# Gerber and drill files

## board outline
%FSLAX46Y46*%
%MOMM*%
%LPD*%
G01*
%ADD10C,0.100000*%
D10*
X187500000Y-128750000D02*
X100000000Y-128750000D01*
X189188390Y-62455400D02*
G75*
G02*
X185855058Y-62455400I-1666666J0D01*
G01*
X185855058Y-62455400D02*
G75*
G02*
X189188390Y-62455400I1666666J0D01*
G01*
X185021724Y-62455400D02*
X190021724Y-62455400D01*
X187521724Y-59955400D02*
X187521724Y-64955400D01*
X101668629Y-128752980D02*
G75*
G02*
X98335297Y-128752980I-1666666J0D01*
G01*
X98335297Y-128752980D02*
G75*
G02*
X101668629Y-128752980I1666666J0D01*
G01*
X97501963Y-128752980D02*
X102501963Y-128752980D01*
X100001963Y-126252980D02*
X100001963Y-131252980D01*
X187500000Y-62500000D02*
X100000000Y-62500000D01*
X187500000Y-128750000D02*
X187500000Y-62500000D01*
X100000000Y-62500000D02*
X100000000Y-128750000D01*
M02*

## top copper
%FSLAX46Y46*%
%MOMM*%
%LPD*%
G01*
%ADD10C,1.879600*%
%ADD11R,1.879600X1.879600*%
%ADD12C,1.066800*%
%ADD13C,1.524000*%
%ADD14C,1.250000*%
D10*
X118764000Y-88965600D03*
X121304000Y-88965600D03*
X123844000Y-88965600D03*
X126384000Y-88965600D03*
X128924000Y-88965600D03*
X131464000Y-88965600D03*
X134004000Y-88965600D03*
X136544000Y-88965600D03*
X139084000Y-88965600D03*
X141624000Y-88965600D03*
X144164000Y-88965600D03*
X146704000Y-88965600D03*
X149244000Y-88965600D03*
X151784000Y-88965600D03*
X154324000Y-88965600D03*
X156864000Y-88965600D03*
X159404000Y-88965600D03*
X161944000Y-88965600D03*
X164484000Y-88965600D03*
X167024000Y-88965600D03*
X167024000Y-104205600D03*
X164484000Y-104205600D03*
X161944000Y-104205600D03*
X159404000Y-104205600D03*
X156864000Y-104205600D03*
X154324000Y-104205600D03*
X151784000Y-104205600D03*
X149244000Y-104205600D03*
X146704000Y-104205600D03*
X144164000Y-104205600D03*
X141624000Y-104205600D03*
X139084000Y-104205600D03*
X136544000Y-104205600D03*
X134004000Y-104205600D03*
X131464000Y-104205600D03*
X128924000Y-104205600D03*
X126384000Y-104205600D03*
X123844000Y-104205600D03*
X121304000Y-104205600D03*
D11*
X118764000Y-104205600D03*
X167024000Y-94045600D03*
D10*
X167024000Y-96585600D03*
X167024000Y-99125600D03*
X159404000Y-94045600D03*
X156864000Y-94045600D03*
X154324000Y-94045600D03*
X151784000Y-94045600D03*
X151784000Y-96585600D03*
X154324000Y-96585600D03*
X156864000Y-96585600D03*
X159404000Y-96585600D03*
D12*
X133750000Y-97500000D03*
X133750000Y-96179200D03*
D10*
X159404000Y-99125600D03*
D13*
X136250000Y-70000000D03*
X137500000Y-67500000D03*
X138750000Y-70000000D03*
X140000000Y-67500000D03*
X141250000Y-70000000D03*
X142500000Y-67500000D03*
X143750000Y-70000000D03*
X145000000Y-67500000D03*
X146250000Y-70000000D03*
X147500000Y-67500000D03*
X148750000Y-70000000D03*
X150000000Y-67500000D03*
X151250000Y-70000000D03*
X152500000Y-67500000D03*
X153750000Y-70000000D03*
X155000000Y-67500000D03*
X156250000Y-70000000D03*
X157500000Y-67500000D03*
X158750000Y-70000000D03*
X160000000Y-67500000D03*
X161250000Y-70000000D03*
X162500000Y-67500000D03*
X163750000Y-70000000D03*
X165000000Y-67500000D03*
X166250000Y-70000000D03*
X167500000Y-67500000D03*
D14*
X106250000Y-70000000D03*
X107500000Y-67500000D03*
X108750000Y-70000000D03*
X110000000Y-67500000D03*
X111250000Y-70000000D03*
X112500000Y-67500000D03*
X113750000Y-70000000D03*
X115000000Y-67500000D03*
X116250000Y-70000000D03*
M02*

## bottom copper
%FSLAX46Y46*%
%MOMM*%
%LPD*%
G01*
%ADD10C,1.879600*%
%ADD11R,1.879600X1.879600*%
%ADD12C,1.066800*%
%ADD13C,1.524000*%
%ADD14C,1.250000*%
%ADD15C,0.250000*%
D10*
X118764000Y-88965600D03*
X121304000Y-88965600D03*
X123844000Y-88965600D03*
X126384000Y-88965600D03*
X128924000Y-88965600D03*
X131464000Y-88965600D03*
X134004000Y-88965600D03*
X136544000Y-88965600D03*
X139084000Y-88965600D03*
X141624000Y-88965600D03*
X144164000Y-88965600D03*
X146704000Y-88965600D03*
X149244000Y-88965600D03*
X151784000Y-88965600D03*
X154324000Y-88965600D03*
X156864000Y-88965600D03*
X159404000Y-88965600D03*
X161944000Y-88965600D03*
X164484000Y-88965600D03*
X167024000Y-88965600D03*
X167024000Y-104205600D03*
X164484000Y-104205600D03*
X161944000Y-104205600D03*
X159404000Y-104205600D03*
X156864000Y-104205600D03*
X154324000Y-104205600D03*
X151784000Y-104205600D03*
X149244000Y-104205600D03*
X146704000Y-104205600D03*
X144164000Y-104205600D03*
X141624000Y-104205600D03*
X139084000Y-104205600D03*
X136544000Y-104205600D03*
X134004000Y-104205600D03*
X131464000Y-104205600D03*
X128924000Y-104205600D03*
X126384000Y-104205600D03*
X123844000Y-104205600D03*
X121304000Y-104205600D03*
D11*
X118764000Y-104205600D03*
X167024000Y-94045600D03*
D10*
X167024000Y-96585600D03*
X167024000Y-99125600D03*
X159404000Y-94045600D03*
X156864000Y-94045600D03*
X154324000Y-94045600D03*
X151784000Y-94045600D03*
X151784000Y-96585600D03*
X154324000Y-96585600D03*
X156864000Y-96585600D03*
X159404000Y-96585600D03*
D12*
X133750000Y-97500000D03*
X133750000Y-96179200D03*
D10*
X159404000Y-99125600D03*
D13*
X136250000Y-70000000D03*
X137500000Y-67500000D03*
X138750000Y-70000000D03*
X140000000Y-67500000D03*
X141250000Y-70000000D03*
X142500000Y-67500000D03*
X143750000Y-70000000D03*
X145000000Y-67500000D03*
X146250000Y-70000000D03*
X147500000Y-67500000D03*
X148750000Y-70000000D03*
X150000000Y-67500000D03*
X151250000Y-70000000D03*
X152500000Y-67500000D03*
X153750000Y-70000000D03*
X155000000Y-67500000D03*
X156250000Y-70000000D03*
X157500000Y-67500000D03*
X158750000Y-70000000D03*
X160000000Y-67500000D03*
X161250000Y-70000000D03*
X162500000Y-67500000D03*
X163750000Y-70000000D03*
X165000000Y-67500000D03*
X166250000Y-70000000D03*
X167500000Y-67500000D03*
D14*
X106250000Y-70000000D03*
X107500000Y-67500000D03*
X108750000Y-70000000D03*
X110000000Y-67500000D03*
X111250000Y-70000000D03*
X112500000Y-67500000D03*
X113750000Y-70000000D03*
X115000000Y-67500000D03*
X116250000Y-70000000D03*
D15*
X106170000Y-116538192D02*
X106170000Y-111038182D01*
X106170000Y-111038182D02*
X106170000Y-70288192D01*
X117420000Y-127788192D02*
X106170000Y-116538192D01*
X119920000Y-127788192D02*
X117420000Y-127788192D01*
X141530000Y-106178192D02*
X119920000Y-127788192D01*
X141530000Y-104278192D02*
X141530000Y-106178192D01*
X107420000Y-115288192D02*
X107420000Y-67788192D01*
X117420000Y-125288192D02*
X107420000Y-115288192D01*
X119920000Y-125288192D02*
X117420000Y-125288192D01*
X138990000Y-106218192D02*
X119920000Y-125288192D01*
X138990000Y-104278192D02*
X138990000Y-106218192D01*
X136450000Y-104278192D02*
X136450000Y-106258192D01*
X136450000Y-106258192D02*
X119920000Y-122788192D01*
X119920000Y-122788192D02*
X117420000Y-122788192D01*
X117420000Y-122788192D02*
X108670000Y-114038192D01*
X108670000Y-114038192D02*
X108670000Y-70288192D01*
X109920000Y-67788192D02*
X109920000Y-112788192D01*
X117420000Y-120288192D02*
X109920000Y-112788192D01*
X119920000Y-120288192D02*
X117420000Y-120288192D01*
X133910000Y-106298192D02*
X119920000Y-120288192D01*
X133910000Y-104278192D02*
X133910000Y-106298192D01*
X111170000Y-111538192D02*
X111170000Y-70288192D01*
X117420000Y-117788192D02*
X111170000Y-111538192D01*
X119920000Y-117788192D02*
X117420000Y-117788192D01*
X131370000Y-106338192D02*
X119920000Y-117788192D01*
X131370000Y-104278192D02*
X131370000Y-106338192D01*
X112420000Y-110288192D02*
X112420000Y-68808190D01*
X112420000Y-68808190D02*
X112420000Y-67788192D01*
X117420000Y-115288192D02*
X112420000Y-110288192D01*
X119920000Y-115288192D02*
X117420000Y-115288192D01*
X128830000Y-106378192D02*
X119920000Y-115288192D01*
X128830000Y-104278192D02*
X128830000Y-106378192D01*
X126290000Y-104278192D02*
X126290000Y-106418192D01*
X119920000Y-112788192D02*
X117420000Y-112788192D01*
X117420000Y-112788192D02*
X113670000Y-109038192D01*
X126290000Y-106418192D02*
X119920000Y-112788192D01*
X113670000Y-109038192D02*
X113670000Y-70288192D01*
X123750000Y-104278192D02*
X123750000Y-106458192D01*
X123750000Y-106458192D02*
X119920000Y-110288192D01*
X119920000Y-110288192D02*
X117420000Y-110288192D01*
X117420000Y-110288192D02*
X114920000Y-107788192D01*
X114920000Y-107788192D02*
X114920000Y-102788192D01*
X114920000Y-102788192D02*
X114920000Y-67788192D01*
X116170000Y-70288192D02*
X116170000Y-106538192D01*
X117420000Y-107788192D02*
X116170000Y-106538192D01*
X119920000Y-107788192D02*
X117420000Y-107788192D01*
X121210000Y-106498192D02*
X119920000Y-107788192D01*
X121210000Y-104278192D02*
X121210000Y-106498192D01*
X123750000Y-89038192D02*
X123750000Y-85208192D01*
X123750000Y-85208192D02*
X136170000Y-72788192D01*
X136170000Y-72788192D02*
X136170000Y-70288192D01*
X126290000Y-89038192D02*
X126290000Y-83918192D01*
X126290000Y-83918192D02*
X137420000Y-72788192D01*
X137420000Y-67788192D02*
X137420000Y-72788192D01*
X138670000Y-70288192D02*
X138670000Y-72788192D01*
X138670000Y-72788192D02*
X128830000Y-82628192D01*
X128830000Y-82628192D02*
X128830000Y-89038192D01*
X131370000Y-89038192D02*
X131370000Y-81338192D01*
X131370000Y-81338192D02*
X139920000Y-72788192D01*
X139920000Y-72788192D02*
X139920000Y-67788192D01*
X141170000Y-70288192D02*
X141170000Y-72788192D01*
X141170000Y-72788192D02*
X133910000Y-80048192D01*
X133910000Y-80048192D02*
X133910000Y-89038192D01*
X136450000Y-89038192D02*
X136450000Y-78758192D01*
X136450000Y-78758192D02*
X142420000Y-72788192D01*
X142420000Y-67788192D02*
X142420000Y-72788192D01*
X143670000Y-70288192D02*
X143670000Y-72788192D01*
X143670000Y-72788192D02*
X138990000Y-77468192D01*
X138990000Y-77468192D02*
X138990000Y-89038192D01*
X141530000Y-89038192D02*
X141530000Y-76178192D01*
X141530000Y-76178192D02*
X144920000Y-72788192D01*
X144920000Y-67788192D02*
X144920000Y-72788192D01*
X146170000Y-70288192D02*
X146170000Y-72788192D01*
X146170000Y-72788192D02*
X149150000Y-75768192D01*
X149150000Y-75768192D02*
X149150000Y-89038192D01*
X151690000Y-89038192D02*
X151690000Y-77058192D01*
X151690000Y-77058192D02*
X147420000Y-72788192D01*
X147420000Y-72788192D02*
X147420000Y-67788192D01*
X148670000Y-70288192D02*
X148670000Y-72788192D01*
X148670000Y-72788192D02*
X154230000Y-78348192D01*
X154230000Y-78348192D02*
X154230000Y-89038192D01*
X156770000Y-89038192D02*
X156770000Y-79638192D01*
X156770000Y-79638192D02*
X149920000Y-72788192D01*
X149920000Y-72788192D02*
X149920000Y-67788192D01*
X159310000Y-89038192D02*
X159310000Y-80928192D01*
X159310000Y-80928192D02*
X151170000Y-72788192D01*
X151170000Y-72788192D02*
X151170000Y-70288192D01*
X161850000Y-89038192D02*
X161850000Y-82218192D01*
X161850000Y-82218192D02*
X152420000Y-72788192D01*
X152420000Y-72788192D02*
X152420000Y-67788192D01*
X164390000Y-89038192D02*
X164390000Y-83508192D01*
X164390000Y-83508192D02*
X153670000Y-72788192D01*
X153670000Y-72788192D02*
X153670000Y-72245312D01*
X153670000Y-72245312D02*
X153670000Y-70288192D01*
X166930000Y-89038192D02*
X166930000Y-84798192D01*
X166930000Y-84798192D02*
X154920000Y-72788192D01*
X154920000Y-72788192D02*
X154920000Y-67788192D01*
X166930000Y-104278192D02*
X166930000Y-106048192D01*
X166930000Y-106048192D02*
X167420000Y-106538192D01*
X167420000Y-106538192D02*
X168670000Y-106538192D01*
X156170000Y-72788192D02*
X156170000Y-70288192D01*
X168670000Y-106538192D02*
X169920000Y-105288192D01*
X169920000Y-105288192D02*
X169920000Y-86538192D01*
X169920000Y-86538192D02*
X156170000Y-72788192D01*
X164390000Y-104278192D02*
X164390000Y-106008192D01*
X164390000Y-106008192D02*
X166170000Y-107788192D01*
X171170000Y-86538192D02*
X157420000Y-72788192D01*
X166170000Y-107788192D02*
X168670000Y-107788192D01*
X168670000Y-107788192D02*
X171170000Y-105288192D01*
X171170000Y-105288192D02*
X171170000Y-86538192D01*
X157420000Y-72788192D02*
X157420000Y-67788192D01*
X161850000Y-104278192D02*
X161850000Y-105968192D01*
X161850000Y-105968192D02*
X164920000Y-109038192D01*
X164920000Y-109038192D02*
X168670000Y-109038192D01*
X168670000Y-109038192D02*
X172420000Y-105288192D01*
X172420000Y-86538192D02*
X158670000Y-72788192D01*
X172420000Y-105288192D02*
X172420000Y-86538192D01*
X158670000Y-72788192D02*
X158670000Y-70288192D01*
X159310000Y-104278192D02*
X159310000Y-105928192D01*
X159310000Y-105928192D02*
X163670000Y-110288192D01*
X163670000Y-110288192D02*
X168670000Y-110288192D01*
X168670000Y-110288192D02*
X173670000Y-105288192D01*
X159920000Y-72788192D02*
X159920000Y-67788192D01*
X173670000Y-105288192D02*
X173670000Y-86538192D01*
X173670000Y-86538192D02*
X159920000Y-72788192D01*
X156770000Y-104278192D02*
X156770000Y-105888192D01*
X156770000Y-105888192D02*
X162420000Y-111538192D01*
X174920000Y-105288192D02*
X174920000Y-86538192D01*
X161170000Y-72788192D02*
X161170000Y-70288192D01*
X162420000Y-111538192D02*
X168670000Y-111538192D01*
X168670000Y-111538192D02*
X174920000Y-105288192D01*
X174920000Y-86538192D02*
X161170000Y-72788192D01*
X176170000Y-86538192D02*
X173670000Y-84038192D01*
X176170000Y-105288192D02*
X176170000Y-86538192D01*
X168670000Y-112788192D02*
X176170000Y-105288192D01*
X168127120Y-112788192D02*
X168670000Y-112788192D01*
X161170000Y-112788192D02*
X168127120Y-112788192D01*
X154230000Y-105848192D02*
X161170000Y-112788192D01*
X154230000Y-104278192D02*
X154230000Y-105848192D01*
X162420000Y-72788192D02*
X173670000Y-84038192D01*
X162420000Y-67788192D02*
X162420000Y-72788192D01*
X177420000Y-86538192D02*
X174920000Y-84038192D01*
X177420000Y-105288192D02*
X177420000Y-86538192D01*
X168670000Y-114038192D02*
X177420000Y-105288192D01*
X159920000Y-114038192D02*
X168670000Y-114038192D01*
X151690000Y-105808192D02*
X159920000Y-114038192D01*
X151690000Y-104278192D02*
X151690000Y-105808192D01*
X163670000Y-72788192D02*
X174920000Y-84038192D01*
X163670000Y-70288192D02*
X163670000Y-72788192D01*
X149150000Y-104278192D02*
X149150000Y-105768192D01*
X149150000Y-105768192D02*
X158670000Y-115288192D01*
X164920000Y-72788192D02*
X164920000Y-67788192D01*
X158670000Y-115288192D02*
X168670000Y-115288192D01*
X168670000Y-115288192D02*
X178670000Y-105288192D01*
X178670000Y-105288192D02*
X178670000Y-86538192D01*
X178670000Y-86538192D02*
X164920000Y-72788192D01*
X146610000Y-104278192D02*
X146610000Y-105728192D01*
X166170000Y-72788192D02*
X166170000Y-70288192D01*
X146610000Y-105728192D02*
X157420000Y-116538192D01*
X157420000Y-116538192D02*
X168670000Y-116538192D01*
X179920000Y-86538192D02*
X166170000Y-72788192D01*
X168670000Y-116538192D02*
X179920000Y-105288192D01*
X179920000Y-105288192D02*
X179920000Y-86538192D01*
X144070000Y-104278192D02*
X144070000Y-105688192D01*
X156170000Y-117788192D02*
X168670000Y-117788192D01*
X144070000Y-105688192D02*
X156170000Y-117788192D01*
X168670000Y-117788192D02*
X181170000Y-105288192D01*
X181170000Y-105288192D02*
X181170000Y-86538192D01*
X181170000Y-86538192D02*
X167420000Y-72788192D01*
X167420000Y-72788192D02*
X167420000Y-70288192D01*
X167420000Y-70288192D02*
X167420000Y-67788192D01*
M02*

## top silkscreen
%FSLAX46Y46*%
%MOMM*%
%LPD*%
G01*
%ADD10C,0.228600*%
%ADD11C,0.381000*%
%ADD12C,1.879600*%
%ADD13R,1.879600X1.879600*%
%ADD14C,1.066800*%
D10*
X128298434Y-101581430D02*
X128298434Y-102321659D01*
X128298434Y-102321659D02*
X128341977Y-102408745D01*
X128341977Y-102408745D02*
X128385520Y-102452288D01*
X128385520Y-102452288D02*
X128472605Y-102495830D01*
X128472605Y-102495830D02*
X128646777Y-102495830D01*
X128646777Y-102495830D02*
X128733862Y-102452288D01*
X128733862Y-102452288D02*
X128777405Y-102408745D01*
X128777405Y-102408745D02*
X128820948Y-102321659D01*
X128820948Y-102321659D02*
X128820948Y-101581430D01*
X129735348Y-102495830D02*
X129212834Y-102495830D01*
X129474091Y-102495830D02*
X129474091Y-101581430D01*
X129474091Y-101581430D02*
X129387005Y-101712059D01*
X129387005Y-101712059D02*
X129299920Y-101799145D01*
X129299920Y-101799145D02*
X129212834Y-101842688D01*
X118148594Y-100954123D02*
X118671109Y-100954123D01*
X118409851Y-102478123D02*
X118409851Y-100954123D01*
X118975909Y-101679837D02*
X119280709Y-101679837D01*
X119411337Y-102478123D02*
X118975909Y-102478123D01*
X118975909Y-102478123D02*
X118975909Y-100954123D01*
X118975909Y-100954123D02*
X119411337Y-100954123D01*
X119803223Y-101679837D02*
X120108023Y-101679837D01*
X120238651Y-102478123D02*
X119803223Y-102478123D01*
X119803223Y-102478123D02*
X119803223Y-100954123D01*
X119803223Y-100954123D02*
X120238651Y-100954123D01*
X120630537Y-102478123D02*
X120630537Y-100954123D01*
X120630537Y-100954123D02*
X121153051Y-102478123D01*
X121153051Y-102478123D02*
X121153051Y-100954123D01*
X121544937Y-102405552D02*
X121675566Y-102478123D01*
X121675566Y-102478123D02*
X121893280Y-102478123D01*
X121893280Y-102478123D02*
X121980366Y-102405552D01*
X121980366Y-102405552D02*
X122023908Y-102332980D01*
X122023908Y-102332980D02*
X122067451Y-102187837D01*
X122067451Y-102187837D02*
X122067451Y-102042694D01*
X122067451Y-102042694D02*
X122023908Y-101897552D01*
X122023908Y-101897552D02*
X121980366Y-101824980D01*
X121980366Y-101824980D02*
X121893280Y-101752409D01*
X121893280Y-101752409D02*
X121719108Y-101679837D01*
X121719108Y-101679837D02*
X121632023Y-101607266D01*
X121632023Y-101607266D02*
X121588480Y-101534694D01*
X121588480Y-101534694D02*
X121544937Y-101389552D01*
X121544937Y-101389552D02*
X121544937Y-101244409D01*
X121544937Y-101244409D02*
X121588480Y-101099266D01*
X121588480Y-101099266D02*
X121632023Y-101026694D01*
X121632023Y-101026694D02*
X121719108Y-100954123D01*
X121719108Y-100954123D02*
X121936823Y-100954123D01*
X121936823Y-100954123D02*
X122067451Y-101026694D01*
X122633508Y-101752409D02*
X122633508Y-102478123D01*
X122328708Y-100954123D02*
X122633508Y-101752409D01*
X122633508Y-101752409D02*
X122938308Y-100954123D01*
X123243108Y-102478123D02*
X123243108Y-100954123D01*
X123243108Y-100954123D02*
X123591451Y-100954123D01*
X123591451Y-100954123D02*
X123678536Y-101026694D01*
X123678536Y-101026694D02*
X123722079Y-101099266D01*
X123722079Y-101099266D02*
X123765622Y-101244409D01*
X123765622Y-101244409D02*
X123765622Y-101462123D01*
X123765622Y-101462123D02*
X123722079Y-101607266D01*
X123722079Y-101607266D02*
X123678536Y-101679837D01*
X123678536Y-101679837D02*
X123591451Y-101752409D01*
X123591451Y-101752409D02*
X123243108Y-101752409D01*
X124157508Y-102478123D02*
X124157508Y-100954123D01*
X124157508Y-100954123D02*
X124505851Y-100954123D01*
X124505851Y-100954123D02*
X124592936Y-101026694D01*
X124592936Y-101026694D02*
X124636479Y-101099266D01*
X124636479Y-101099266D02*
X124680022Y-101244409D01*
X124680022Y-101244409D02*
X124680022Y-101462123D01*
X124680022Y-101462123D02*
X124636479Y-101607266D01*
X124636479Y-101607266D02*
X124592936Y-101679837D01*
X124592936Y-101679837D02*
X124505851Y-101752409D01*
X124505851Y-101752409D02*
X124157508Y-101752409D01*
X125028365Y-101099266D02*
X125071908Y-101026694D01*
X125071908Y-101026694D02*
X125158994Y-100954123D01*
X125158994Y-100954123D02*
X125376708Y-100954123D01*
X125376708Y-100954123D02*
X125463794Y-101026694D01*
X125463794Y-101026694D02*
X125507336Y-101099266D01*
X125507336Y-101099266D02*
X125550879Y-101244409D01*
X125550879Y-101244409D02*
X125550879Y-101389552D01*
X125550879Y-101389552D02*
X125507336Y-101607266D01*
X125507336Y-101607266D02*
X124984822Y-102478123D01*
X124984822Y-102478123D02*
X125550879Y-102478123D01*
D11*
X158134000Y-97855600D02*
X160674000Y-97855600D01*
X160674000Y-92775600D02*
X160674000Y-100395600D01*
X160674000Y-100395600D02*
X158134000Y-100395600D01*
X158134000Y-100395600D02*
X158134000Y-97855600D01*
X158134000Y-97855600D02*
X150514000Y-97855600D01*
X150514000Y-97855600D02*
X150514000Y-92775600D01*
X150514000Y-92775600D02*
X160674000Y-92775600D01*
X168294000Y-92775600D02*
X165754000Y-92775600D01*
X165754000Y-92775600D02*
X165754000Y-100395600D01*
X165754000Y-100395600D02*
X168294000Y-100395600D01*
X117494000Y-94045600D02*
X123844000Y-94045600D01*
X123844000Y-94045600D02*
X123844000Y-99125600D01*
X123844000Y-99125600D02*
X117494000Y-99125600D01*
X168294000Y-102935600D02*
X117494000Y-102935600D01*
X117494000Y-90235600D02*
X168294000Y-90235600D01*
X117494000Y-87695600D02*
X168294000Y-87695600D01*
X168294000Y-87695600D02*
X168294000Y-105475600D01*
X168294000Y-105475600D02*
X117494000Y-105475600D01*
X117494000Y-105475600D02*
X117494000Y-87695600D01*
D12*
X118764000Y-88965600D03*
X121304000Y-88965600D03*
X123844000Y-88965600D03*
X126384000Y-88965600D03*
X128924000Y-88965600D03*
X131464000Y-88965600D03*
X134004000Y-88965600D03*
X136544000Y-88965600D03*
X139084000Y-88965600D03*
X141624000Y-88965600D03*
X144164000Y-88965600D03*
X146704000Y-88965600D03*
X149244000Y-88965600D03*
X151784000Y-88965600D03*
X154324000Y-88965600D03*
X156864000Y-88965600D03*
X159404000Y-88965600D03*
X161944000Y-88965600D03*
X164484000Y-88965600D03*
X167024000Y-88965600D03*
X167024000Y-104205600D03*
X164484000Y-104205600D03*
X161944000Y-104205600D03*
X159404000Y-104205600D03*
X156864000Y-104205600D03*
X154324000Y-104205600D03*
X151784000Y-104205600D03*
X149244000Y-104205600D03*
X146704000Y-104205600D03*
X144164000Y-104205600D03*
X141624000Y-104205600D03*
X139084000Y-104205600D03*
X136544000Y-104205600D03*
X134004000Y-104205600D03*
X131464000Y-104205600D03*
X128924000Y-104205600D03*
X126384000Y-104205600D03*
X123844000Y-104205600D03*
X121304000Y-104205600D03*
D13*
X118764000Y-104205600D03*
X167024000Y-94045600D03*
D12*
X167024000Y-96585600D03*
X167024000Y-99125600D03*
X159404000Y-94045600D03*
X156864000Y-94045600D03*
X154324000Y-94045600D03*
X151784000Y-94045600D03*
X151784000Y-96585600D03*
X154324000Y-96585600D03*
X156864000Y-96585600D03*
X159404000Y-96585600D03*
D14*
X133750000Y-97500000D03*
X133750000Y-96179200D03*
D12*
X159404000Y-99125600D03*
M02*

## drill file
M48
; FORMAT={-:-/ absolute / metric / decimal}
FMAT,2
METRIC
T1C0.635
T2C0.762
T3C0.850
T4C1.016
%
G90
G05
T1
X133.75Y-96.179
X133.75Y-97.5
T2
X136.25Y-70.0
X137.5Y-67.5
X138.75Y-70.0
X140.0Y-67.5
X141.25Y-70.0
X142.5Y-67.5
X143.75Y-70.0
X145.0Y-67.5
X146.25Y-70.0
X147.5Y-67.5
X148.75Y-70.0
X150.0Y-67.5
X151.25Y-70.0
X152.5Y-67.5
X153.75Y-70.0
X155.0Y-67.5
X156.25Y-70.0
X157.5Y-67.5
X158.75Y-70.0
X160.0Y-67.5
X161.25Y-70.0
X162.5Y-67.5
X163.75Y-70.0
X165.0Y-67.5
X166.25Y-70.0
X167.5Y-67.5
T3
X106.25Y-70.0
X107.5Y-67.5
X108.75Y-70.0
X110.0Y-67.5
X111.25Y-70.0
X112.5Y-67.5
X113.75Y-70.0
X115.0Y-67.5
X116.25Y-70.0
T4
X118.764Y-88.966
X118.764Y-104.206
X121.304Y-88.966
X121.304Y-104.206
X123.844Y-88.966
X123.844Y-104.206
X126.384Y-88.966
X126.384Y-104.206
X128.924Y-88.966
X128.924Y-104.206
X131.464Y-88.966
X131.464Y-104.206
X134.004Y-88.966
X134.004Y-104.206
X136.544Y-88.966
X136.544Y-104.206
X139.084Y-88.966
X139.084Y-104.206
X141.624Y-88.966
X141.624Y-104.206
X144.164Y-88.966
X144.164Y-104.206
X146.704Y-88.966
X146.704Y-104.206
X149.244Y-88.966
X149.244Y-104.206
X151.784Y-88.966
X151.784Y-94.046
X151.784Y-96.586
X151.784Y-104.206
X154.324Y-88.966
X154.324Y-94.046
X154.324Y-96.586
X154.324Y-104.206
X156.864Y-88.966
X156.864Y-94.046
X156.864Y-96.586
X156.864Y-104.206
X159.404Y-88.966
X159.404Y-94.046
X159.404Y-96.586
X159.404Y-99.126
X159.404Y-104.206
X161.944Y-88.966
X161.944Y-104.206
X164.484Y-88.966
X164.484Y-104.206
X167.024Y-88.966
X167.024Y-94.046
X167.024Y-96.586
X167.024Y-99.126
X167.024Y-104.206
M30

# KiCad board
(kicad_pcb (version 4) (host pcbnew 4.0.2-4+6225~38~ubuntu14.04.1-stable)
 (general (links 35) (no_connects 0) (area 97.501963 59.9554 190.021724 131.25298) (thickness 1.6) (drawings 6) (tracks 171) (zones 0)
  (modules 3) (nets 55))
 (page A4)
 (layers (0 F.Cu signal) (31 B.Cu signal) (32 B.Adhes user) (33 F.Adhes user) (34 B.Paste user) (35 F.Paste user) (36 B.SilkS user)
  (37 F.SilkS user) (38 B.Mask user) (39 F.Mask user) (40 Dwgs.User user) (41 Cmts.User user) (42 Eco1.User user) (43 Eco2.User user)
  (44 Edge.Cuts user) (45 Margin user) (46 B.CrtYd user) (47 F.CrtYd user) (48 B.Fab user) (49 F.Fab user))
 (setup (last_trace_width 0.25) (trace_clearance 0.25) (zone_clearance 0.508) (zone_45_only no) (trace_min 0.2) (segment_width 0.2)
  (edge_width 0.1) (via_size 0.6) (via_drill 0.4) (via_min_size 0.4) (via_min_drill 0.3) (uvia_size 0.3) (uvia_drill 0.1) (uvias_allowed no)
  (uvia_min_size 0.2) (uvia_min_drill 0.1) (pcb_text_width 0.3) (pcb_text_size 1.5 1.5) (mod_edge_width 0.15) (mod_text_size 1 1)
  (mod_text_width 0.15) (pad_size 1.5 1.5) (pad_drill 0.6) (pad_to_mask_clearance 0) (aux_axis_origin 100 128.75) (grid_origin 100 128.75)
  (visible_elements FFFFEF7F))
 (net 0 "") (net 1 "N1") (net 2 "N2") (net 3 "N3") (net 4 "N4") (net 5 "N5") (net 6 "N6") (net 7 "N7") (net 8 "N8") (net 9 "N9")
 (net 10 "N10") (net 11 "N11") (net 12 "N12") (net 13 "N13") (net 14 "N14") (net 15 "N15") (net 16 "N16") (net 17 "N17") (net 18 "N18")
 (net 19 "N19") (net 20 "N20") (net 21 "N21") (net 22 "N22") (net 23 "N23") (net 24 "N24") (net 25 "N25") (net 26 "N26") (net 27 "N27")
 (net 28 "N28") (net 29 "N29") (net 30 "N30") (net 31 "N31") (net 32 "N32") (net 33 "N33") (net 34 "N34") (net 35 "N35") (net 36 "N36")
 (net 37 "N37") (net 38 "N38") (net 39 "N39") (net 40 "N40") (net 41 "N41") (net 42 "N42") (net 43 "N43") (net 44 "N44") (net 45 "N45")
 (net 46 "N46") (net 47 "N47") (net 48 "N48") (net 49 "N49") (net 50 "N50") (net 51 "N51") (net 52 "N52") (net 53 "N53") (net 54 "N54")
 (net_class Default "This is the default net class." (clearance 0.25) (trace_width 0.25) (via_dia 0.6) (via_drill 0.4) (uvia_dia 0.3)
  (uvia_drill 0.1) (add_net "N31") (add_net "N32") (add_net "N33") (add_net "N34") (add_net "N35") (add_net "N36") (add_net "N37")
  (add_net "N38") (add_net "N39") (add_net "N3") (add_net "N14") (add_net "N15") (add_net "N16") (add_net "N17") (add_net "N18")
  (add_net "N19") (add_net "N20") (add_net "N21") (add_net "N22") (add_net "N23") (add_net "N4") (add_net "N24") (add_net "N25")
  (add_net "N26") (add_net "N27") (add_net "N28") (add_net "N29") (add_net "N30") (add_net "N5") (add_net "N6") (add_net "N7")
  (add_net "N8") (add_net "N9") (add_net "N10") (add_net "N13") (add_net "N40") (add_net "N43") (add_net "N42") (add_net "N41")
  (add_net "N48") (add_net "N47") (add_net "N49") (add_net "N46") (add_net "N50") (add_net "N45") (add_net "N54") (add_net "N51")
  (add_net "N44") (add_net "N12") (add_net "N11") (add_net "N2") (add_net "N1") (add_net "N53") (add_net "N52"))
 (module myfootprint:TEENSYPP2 (layer F.Cu) (at 142.894 96.5856)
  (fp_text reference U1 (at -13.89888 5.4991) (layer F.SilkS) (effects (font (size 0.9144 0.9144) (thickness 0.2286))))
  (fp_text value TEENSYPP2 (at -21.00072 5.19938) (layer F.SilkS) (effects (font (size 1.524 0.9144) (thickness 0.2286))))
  (fp_line (start 15.24 1.27) (end 17.78 1.27) (layer F.SilkS) (width 0.381))
  (fp_line (start 17.78 -3.81) (end 17.78 3.81) (layer F.SilkS) (width 0.381))
  (fp_line (start 17.78 3.81) (end 15.24 3.81) (layer F.SilkS) (width 0.381))
  (fp_line (start 15.24 3.81) (end 15.24 1.27) (layer F.SilkS) (width 0.381))
  (fp_line (start 15.24 1.27) (end 7.62 1.27) (layer F.SilkS) (width 0.381))
  (fp_line (start 7.62 1.27) (end 7.62 -3.81) (layer F.SilkS) (width 0.381))
  (fp_line (start 7.62 -3.81) (end 17.78 -3.81) (layer F.SilkS) (width 0.381))
  (fp_line (start 25.4 -3.81) (end 22.86 -3.81) (layer F.SilkS) (width 0.381))
  (fp_line (start 22.86 -3.81) (end 22.86 3.81) (layer F.SilkS) (width 0.381))
  (fp_line (start 22.86 3.81) (end 25.4 3.81) (layer F.SilkS) (width 0.381))
  (fp_line (start -25.4 -2.54) (end -19.05 -2.54) (layer F.SilkS) (width 0.381))
  (fp_line (start -19.05 -2.54) (end -19.05 2.54) (layer F.SilkS) (width 0.381))
  (fp_line (start -19.05 2.54) (end -25.4 2.54) (layer F.SilkS) (width 0.381))
  (fp_line (start 25.4 6.35) (end -25.4 6.35) (layer F.SilkS) (width 0.381))
  (fp_line (start -25.4 -6.35) (end 25.4 -6.35) (layer F.SilkS) (width 0.381))
  (fp_line (start -25.4 -8.89) (end 25.4 -8.89) (layer F.SilkS) (width 0.381))
  (fp_line (start 25.4 -8.89) (end 25.4 8.89) (layer F.SilkS) (width 0.381))
  (fp_line (start 25.4 8.89) (end -25.4 8.89) (layer F.SilkS) (width 0.381))
  (fp_line (start -25.4 8.89) (end -25.4 -8.89) (layer F.SilkS) (width 0.381))
  (pad 52 thru_hole circle (at -24.13 -7.62) (size 1.8796 1.8796) (drill 1.016) (layers *.Cu *.Mask F.SilkS) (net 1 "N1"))
  (pad 51 thru_hole circle (at -21.59 -7.62) (size 1.8796 1.8796) (drill 1.016) (layers *.Cu *.Mask F.SilkS) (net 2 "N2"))
  (pad 50 thru_hole circle (at -19.05 -7.62) (size 1.8796 1.8796) (drill 1.016) (layers *.Cu *.Mask F.SilkS) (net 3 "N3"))
  (pad 49 thru_hole circle (at -16.51 -7.62) (size 1.8796 1.8796) (drill 1.016) (layers *.Cu *.Mask F.SilkS) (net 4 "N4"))
  (pad 48 thru_hole circle (at -13.97 -7.62) (size 1.8796 1.8796) (drill 1.016) (layers *.Cu *.Mask F.SilkS) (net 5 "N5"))
  (pad 47 thru_hole circle (at -11.43 -7.62) (size 1.8796 1.8796) (drill 1.016) (layers *.Cu *.Mask F.SilkS) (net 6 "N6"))
  (pad 46 thru_hole circle (at -8.89 -7.62) (size 1.8796 1.8796) (drill 1.016) (layers *.Cu *.Mask F.SilkS) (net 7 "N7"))
  (pad 45 thru_hole circle (at -6.35 -7.62) (size 1.8796 1.8796) (drill 1.016) (layers *.Cu *.Mask F.SilkS) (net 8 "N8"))
  (pad 44 thru_hole circle (at -3.81 -7.62) (size 1.8796 1.8796) (drill 1.016) (layers *.Cu *.Mask F.SilkS) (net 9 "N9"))
  (pad 43 thru_hole circle (at -1.27 -7.62) (size 1.8796 1.8796) (drill 1.016) (layers *.Cu *.Mask F.SilkS) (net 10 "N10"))
  (pad 42 thru_hole circle (at 1.27 -7.62) (size 1.8796 1.8796) (drill 1.016) (layers *.Cu *.Mask F.SilkS) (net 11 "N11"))
  (pad 41 thru_hole circle (at 3.81 -7.62) (size 1.8796 1.8796) (drill 1.016) (layers *.Cu *.Mask F.SilkS) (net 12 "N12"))
  (pad 40 thru_hole circle (at 6.35 -7.62) (size 1.8796 1.8796) (drill 1.016) (layers *.Cu *.Mask F.SilkS) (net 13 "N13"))
  (pad 39 thru_hole circle (at 8.89 -7.62) (size 1.8796 1.8796) (drill 1.016) (layers *.Cu *.Mask F.SilkS) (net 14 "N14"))
  (pad 38 thru_hole circle (at 11.43 -7.62) (size 1.8796 1.8796) (drill 1.016) (layers *.Cu *.Mask F.SilkS) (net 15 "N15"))
  (pad 37 thru_hole circle (at 13.97 -7.62) (size 1.8796 1.8796) (drill 1.016) (layers *.Cu *.Mask F.SilkS) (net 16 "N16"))
  (pad 36 thru_hole circle (at 16.51 -7.62) (size 1.8796 1.8796) (drill 1.016) (layers *.Cu *.Mask F.SilkS) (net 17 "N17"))
  (pad 35 thru_hole circle (at 19.05 -7.62) (size 1.8796 1.8796) (drill 1.016) (layers *.Cu *.Mask F.SilkS) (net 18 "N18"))
  (pad 34 thru_hole circle (at 21.59 -7.62) (size 1.8796 1.8796) (drill 1.016) (layers *.Cu *.Mask F.SilkS) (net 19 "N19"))
  (pad 33 thru_hole circle (at 24.13 -7.62) (size 1.8796 1.8796) (drill 1.016) (layers *.Cu *.Mask F.SilkS) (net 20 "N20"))
  (pad 20 thru_hole circle (at 24.13 7.62) (size 1.8796 1.8796) (drill 1.016) (layers *.Cu *.Mask F.SilkS) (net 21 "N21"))
  (pad 19 thru_hole circle (at 21.59 7.62) (size 1.8796 1.8796) (drill 1.016) (layers *.Cu *.Mask F.SilkS) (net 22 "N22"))
  (pad 18 thru_hole circle (at 19.05 7.62) (size 1.8796 1.8796) (drill 1.016) (layers *.Cu *.Mask F.SilkS) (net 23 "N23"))
  (pad 17 thru_hole circle (at 16.51 7.62) (size 1.8796 1.8796) (drill 1.016) (layers *.Cu *.Mask F.SilkS) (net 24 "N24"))
  (pad 16 thru_hole circle (at 13.97 7.62) (size 1.8796 1.8796) (drill 1.016) (layers *.Cu *.Mask F.SilkS) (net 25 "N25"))
  (pad 15 thru_hole circle (at 11.43 7.62) (size 1.8796 1.8796) (drill 1.016) (layers *.Cu *.Mask F.SilkS) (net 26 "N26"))
  (pad 14 thru_hole circle (at 8.89 7.62) (size 1.8796 1.8796) (drill 1.016) (layers *.Cu *.Mask F.SilkS) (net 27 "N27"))
  (pad 13 thru_hole circle (at 6.35 7.62) (size 1.8796 1.8796) (drill 1.016) (layers *.Cu *.Mask F.SilkS) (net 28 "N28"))
  (pad 12 thru_hole circle (at 3.81 7.62) (size 1.8796 1.8796) (drill 1.016) (layers *.Cu *.Mask F.SilkS) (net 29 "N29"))
  (pad 11 thru_hole circle (at 1.27 7.62) (size 1.8796 1.8796) (drill 1.016) (layers *.Cu *.Mask F.SilkS) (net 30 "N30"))
  (pad 10 thru_hole circle (at -1.27 7.62) (size 1.8796 1.8796) (drill 1.016) (layers *.Cu *.Mask F.SilkS) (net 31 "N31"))
  (pad 9 thru_hole circle (at -3.81 7.62) (size 1.8796 1.8796) (drill 1.016) (layers *.Cu *.Mask F.SilkS) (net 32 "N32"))
  (pad 8 thru_hole circle (at -6.35 7.62) (size 1.8796 1.8796) (drill 1.016) (layers *.Cu *.Mask F.SilkS) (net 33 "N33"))
  (pad 7 thru_hole circle (at -8.89 7.62) (size 1.8796 1.8796) (drill 1.016) (layers *.Cu *.Mask F.SilkS) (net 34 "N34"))
  (pad 6 thru_hole circle (at -11.43 7.62) (size 1.8796 1.8796) (drill 1.016) (layers *.Cu *.Mask F.SilkS) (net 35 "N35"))
  (pad 5 thru_hole circle (at -13.97 7.62) (size 1.8796 1.8796) (drill 1.016) (layers *.Cu *.Mask F.SilkS) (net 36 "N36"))
  (pad 4 thru_hole circle (at -16.51 7.62) (size 1.8796 1.8796) (drill 1.016) (layers *.Cu *.Mask F.SilkS) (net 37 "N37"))
  (pad 3 thru_hole circle (at -19.05 7.62) (size 1.8796 1.8796) (drill 1.016) (layers *.Cu *.Mask F.SilkS) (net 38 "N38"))
  (pad 2 thru_hole circle (at -21.59 7.62) (size 1.8796 1.8796) (drill 1.016) (layers *.Cu *.Mask F.SilkS) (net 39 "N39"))
  (pad 1 thru_hole rect (at -24.13 7.62) (size 1.8796 1.8796) (drill 1.016) (layers *.Cu *.Mask F.SilkS) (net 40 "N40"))
  (pad 23 thru_hole rect (at 24.13 -2.54) (size 1.8796 1.8796) (drill 1.016) (layers *.Cu *.Mask F.SilkS) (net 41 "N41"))
  (pad 22 thru_hole circle (at 24.13 0) (size 1.8796 1.8796) (drill 1.016) (layers *.Cu *.Mask F.SilkS) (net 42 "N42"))
  (pad 21 thru_hole circle (at 24.13 2.54) (size 1.8796 1.8796) (drill 1.016) (layers *.Cu *.Mask F.SilkS) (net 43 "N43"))
  (pad 32 thru_hole circle (at 16.51 -2.54) (size 1.8796 1.8796) (drill 1.016) (layers *.Cu *.Mask F.SilkS) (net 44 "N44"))
  (pad 29 thru_hole circle (at 13.97 -2.54) (size 1.8796 1.8796) (drill 1.016) (layers *.Cu *.Mask F.SilkS) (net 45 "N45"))
  (pad 27 thru_hole circle (at 11.43 -2.54) (size 1.8796 1.8796) (drill 1.016) (layers *.Cu *.Mask F.SilkS) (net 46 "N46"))
  (pad 25 thru_hole circle (at 8.89 -2.54) (size 1.8796 1.8796) (drill 1.016) (layers *.Cu *.Mask F.SilkS) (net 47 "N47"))
  (pad 24 thru_hole circle (at 8.89 0) (size 1.8796 1.8796) (drill 1.016) (layers *.Cu *.Mask F.SilkS) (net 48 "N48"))
  (pad 26 thru_hole circle (at 11.43 0) (size 1.8796 1.8796) (drill 1.016) (layers *.Cu *.Mask F.SilkS) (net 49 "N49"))
  (pad 28 thru_hole circle (at 13.97 0) (size 1.8796 1.8796) (drill 1.016) (layers *.Cu *.Mask F.SilkS) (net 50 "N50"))
  (pad 31 thru_hole circle (at 16.51 0) (size 1.8796 1.8796) (drill 1.016) (layers *.Cu *.Mask F.SilkS) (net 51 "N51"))
  (pad 54 thru_hole circle (at -9.144 0.9144) (size 1.0668 1.0668) (drill 0.635) (layers *.Cu *.Mask F.SilkS) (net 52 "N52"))
  (pad 53 thru_hole circle (at -9.144 -0.4064) (size 1.0668 1.0668) (drill 0.635) (layers *.Cu *.Mask F.SilkS) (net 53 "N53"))
  (pad 30 thru_hole circle (at 16.51 2.54) (size 1.8796 1.8796) (drill 1.016) (layers *.Cu *.Mask F.SilkS) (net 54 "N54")))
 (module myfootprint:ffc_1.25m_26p (layer B.Cu) (at 151.25 72.5)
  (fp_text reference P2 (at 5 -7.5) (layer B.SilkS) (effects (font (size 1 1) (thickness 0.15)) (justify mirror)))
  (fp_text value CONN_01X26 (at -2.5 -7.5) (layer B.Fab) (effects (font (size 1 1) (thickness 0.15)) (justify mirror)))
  (pad 1 thru_hole circle (at -15 -2.5) (size 1.524 1.524) (drill 0.762) (layers *.Cu *.Mask B.SilkS) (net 3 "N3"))
  (pad 2 thru_hole circle (at -13.75 -5) (size 1.524 1.524) (drill 0.762) (layers *.Cu *.Mask B.SilkS) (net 4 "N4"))
  (pad 3 thru_hole circle (at -12.5 -2.5) (size 1.524 1.524) (drill 0.762) (layers *.Cu *.Mask B.SilkS) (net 5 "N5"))
  (pad 4 thru_hole circle (at -11.25 -5) (size 1.524 1.524) (drill 0.762) (layers *.Cu *.Mask B.SilkS) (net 6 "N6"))
  (pad 5 thru_hole circle (at -10 -2.5) (size 1.524 1.524) (drill 0.762) (layers *.Cu *.Mask B.SilkS) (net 7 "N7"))
  (pad 6 thru_hole circle (at -8.75 -5) (size 1.524 1.524) (drill 0.762) (layers *.Cu *.Mask B.SilkS) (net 8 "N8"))
  (pad 7 thru_hole circle (at -7.5 -2.5) (size 1.524 1.524) (drill 0.762) (layers *.Cu *.Mask B.SilkS) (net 9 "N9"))
  (pad 8 thru_hole circle (at -6.25 -5) (size 1.524 1.524) (drill 0.762) (layers *.Cu *.Mask B.SilkS) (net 10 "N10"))
  (pad 9 thru_hole circle (at -5 -2.5) (size 1.524 1.524) (drill 0.762) (layers *.Cu *.Mask B.SilkS) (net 13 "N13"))
  (pad 10 thru_hole circle (at -3.75 -5) (size 1.524 1.524) (drill 0.762) (layers *.Cu *.Mask B.SilkS) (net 14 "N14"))
  (pad 11 thru_hole circle (at -2.5 -2.5) (size 1.524 1.524) (drill 0.762) (layers *.Cu *.Mask B.SilkS) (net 15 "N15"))
  (pad 12 thru_hole circle (at -1.25 -5) (size 1.524 1.524) (drill 0.762) (layers *.Cu *.Mask B.SilkS) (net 16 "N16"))
  (pad 13 thru_hole circle (at 0 -2.5) (size 1.524 1.524) (drill 0.762) (layers *.Cu *.Mask B.SilkS) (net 17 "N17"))
  (pad 14 thru_hole circle (at 1.25 -5) (size 1.524 1.524) (drill 0.762) (layers *.Cu *.Mask B.SilkS) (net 18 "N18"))
  (pad 15 thru_hole circle (at 2.5 -2.5) (size 1.524 1.524) (drill 0.762) (layers *.Cu *.Mask B.SilkS) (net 19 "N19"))
  (pad 16 thru_hole circle (at 3.75 -5) (size 1.524 1.524) (drill 0.762) (layers *.Cu *.Mask B.SilkS) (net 20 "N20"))
  (pad 17 thru_hole circle (at 5 -2.5) (size 1.524 1.524) (drill 0.762) (layers *.Cu *.Mask B.SilkS) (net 21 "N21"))
  (pad 18 thru_hole circle (at 6.25 -5) (size 1.524 1.524) (drill 0.762) (layers *.Cu *.Mask B.SilkS) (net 22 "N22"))
  (pad 19 thru_hole circle (at 7.5 -2.5) (size 1.524 1.524) (drill 0.762) (layers *.Cu *.Mask B.SilkS) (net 23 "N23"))
  (pad 20 thru_hole circle (at 8.75 -5) (size 1.524 1.524) (drill 0.762) (layers *.Cu *.Mask B.SilkS) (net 24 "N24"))
  (pad 21 thru_hole circle (at 10 -2.5) (size 1.524 1.524) (drill 0.762) (layers *.Cu *.Mask B.SilkS) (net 25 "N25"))
  (pad 22 thru_hole circle (at 11.25 -5) (size 1.524 1.524) (drill 0.762) (layers *.Cu *.Mask B.SilkS) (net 26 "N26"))
  (pad 23 thru_hole circle (at 12.5 -2.5) (size 1.524 1.524) (drill 0.762) (layers *.Cu *.Mask B.SilkS) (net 27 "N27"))
  (pad 24 thru_hole circle (at 13.75 -5) (size 1.524 1.524) (drill 0.762) (layers *.Cu *.Mask B.SilkS) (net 28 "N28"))
  (pad 25 thru_hole circle (at 15 -2.5) (size 1.524 1.524) (drill 0.762) (layers *.Cu *.Mask B.SilkS) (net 29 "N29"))
  (pad 26 thru_hole circle (at 16.25 -5) (size 1.524 1.524) (drill 0.762) (layers *.Cu *.Mask B.SilkS) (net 30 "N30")))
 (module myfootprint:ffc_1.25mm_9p (layer B.Cu) (at 111.25 71.25)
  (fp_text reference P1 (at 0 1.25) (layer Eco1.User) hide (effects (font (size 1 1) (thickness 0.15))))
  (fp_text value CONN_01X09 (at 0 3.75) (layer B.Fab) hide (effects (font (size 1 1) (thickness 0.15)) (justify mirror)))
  (pad 1 thru_hole circle (at -5 -1.25) (size 1.25 1.25) (drill 0.85) (layers *.Cu *.Mask B.SilkS) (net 31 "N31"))
  (pad 2 thru_hole circle (at -3.75 -3.75) (size 1.25 1.25) (drill 0.85) (layers *.Cu *.Mask B.SilkS) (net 32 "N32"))
  (pad 3 thru_hole circle (at -2.5 -1.25) (size 1.25 1.25) (drill 0.85) (layers *.Cu *.Mask B.SilkS) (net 33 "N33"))
  (pad 4 thru_hole circle (at -1.25 -3.75) (size 1.25 1.25) (drill 0.85) (layers *.Cu *.Mask B.SilkS) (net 34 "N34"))
  (pad 5 thru_hole circle (at 0 -1.25) (size 1.25 1.25) (drill 0.85) (layers *.Cu *.Mask B.SilkS) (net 35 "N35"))
  (pad 6 thru_hole circle (at 1.25 -3.75) (size 1.25 1.25) (drill 0.85) (layers *.Cu *.Mask B.SilkS) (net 36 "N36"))
  (pad 7 thru_hole circle (at 2.5 -1.25) (size 1.25 1.25) (drill 0.85) (layers *.Cu *.Mask B.SilkS) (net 37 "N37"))
  (pad 8 thru_hole circle (at 3.75 -3.75) (size 1.25 1.25) (drill 0.85) (layers *.Cu *.Mask B.SilkS) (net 38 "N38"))
  (pad 9 thru_hole circle (at 5 -1.25) (size 1.25 1.25) (drill 0.85) (layers *.Cu *.Mask B.SilkS) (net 39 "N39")))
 (gr_line (start 187.5 128.75) (end 100 128.75) (layer Edge.Cuts) (width 0.1))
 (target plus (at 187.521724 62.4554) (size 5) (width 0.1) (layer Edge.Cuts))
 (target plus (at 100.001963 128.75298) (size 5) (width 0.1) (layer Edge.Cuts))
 (gr_line (start 187.5 62.5) (end 100 62.5) (layer Edge.Cuts) (width 0.1))
 (gr_line (start 187.5 128.75) (end 187.5 62.5) (layer Edge.Cuts) (width 0.1))
 (gr_line (start 100 62.5) (end 100 128.75) (layer Edge.Cuts) (width 0.1))
 (segment (start 106.17 116.538192) (end 106.17 111.038182) (width 0.25) (layer B.Cu) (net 31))
 (segment (start 106.17 111.038182) (end 106.17 70.288192) (width 0.25) (layer B.Cu) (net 31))
 (segment (start 117.42 127.788192) (end 106.17 116.538192) (width 0.25) (layer B.Cu) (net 31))
 (segment (start 119.92 127.788192) (end 117.42 127.788192) (width 0.25) (layer B.Cu) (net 31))
 (segment (start 141.53 106.178192) (end 119.92 127.788192) (width 0.25) (layer B.Cu) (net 31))
 (segment (start 141.53 104.278192) (end 141.53 106.178192) (width 0.25) (layer B.Cu) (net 31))
 (segment (start 107.42 115.288192) (end 107.42 67.788192) (width 0.25) (layer B.Cu) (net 32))
 (segment (start 117.42 125.288192) (end 107.42 115.288192) (width 0.25) (layer B.Cu) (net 32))
 (segment (start 119.92 125.288192) (end 117.42 125.288192) (width 0.25) (layer B.Cu) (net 32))
 (segment (start 138.99 106.218192) (end 119.92 125.288192) (width 0.25) (layer B.Cu) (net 32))
 (segment (start 138.99 104.278192) (end 138.99 106.218192) (width 0.25) (layer B.Cu) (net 32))
 (segment (start 136.45 104.278192) (end 136.45 106.258192) (width 0.25) (layer B.Cu) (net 33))
 (segment (start 136.45 106.258192) (end 119.92 122.788192) (width 0.25) (layer B.Cu) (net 33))
 (segment (start 119.92 122.788192) (end 117.42 122.788192) (width 0.25) (layer B.Cu) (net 33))
 (segment (start 117.42 122.788192) (end 108.67 114.038192) (width 0.25) (layer B.Cu) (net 33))
 (segment (start 108.67 114.038192) (end 108.67 70.288192) (width 0.25) (layer B.Cu) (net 33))
 (segment (start 109.92 67.788192) (end 109.92 112.788192) (width 0.25) (layer B.Cu) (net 34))
 (segment (start 117.42 120.288192) (end 109.92 112.788192) (width 0.25) (layer B.Cu) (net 34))
 (segment (start 119.92 120.288192) (end 117.42 120.288192) (width 0.25) (layer B.Cu) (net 34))
 (segment (start 133.91 106.298192) (end 119.92 120.288192) (width 0.25) (layer B.Cu) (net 34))
 (segment (start 133.91 104.278192) (end 133.91 106.298192) (width 0.25) (layer B.Cu) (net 34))
 (segment (start 111.17 111.538192) (end 111.17 70.288192) (width 0.25) (layer B.Cu) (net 35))
 (segment (start 117.42 117.788192) (end 111.17 111.538192) (width 0.25) (layer B.Cu) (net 35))
 (segment (start 119.92 117.788192) (end 117.42 117.788192) (width 0.25) (layer B.Cu) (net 35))
 (segment (start 131.37 106.338192) (end 119.92 117.788192) (width 0.25) (layer B.Cu) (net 35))
 (segment (start 131.37 104.278192) (end 131.37 106.338192) (width 0.25) (layer B.Cu) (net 35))
 (segment (start 112.42 110.288192) (end 112.42 68.80819) (width 0.25) (layer B.Cu) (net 36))
 (segment (start 112.42 68.80819) (end 112.42 67.788192) (width 0.25) (layer B.Cu) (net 36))
 (segment (start 117.42 115.288192) (end 112.42 110.288192) (width 0.25) (layer B.Cu) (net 36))
 (segment (start 119.92 115.288192) (end 117.42 115.288192) (width 0.25) (layer B.Cu) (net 36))
 (segment (start 128.83 106.378192) (end 119.92 115.288192) (width 0.25) (layer B.Cu) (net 36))
 (segment (start 128.83 104.278192) (end 128.83 106.378192) (width 0.25) (layer B.Cu) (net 36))
 (segment (start 126.29 104.278192) (end 126.29 106.418192) (width 0.25) (layer B.Cu) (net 37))
 (segment (start 119.92 112.788192) (end 117.42 112.788192) (width 0.25) (layer B.Cu) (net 37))
 (segment (start 117.42 112.788192) (end 113.67 109.038192) (width 0.25) (layer B.Cu) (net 37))
 (segment (start 126.29 106.418192) (end 119.92 112.788192) (width 0.25) (layer B.Cu) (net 37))
 (segment (start 113.67 109.038192) (end 113.67 70.288192) (width 0.25) (layer B.Cu) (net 37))
 (segment (start 123.75 104.278192) (end 123.75 106.458192) (width 0.25) (layer B.Cu) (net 38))
 (segment (start 123.75 106.458192) (end 119.92 110.288192) (width 0.25) (layer B.Cu) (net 38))
 (segment (start 119.92 110.288192) (end 117.42 110.288192) (width 0.25) (layer B.Cu) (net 38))
 (segment (start 117.42 110.288192) (end 114.92 107.788192) (width 0.25) (layer B.Cu) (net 38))
 (segment (start 114.92 107.788192) (end 114.92 102.788192) (width 0.25) (layer B.Cu) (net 38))
 (segment (start 114.92 102.788192) (end 114.92 67.788192) (width 0.25) (layer B.Cu) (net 38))
 (segment (start 116.17 70.288192) (end 116.17 106.538192) (width 0.25) (layer B.Cu) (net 39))
 (segment (start 117.42 107.788192) (end 116.17 106.538192) (width 0.25) (layer B.Cu) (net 39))
 (segment (start 119.92 107.788192) (end 117.42 107.788192) (width 0.25) (layer B.Cu) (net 39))
 (segment (start 121.21 106.498192) (end 119.92 107.788192) (width 0.25) (layer B.Cu) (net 39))
 (segment (start 121.21 104.278192) (end 121.21 106.498192) (width 0.25) (layer B.Cu) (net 39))
 (segment (start 123.75 89.038192) (end 123.75 85.208192) (width 0.25) (layer B.Cu) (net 3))
 (segment (start 123.75 85.208192) (end 136.17 72.788192) (width 0.25) (layer B.Cu) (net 3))
 (segment (start 136.17 72.788192) (end 136.17 70.288192) (width 0.25) (layer B.Cu) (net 3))
 (segment (start 126.29 89.038192) (end 126.29 83.918192) (width 0.25) (layer B.Cu) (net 4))
 (segment (start 126.29 83.918192) (end 137.42 72.788192) (width 0.25) (layer B.Cu) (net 4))
 (segment (start 137.42 67.788192) (end 137.42 72.788192) (width 0.25) (layer B.Cu) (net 4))
 (segment (start 138.67 70.288192) (end 138.67 72.788192) (width 0.25) (layer B.Cu) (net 5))
 (segment (start 138.67 72.788192) (end 128.83 82.628192) (width 0.25) (layer B.Cu) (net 5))
 (segment (start 128.83 82.628192) (end 128.83 89.038192) (width 0.25) (layer B.Cu) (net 5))
 (segment (start 131.37 89.038192) (end 131.37 81.338192) (width 0.25) (layer B.Cu) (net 6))
 (segment (start 131.37 81.338192) (end 139.92 72.788192) (width 0.25) (layer B.Cu) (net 6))
 (segment (start 139.92 72.788192) (end 139.92 67.788192) (width 0.25) (layer B.Cu) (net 6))
 (segment (start 141.17 70.288192) (end 141.17 72.788192) (width 0.25) (layer B.Cu) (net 7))
 (segment (start 141.17 72.788192) (end 133.91 80.048192) (width 0.25) (layer B.Cu) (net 7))
 (segment (start 133.91 80.048192) (end 133.91 89.038192) (width 0.25) (layer B.Cu) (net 7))
 (segment (start 136.45 89.038192) (end 136.45 78.758192) (width 0.25) (layer B.Cu) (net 8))
 (segment (start 136.45 78.758192) (end 142.42 72.788192) (width 0.25) (layer B.Cu) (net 8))
 (segment (start 142.42 67.788192) (end 142.42 72.788192) (width 0.25) (layer B.Cu) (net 8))
 (segment (start 143.67 70.288192) (end 143.67 72.788192) (width 0.25) (layer B.Cu) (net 9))
 (segment (start 143.67 72.788192) (end 138.99 77.468192) (width 0.25) (layer B.Cu) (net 9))
 (segment (start 138.99 77.468192) (end 138.99 89.038192) (width 0.25) (layer B.Cu) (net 9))
 (segment (start 141.53 89.038192) (end 141.53 76.178192) (width 0.25) (layer B.Cu) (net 10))
 (segment (start 141.53 76.178192) (end 144.92 72.788192) (width 0.25) (layer B.Cu) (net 10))
 (segment (start 144.92 67.788192) (end 144.92 72.788192) (width 0.25) (layer B.Cu) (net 10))
 (segment (start 146.17 70.288192) (end 146.17 72.788192) (width 0.25) (layer B.Cu) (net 13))
 (segment (start 146.17 72.788192) (end 149.15 75.768192) (width 0.25) (layer B.Cu) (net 13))
 (segment (start 149.15 75.768192) (end 149.15 89.038192) (width 0.25) (layer B.Cu) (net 13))
 (segment (start 151.69 89.038192) (end 151.69 77.058192) (width 0.25) (layer B.Cu) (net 14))
 (segment (start 151.69 77.058192) (end 147.42 72.788192) (width 0.25) (layer B.Cu) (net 14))
 (segment (start 147.42 72.788192) (end 147.42 67.788192) (width 0.25) (layer B.Cu) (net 14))
 (segment (start 148.67 70.288192) (end 148.67 72.788192) (width 0.25) (layer B.Cu) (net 15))
 (segment (start 148.67 72.788192) (end 154.23 78.348192) (width 0.25) (layer B.Cu) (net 15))
 (segment (start 154.23 78.348192) (end 154.23 89.038192) (width 0.25) (layer B.Cu) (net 15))
 (segment (start 156.77 89.038192) (end 156.77 79.638192) (width 0.25) (layer B.Cu) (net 16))
 (segment (start 156.77 79.638192) (end 149.92 72.788192) (width 0.25) (layer B.Cu) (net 16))
 (segment (start 149.92 72.788192) (end 149.92 67.788192) (width 0.25) (layer B.Cu) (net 16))
 (segment (start 159.31 89.038192) (end 159.31 80.928192) (width 0.25) (layer B.Cu) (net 17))
 (segment (start 159.31 80.928192) (end 151.17 72.788192) (width 0.25) (layer B.Cu) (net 17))
 (segment (start 151.17 72.788192) (end 151.17 70.288192) (width 0.25) (layer B.Cu) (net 17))
 (segment (start 161.85 89.038192) (end 161.85 82.218192) (width 0.25) (layer B.Cu) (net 18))
 (segment (start 161.85 82.218192) (end 152.42 72.788192) (width 0.25) (layer B.Cu) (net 18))
 (segment (start 152.42 72.788192) (end 152.42 67.788192) (width 0.25) (layer B.Cu) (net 18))
 (segment (start 164.39 89.038192) (end 164.39 83.508192) (width 0.25) (layer B.Cu) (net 19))
 (segment (start 164.39 83.508192) (end 153.67 72.788192) (width 0.25) (layer B.Cu) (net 19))
 (segment (start 153.67 72.788192) (end 153.67 72.245312) (width 0.25) (layer B.Cu) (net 19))
 (segment (start 153.67 72.245312) (end 153.67 70.288192) (width 0.25) (layer B.Cu) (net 19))
 (segment (start 166.93 89.038192) (end 166.93 84.798192) (width 0.25) (layer B.Cu) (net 20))
 (segment (start 166.93 84.798192) (end 154.92 72.788192) (width 0.25) (layer B.Cu) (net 20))
 (segment (start 154.92 72.788192) (end 154.92 67.788192) (width 0.25) (layer B.Cu) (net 20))
 (segment (start 166.93 104.278192) (end 166.93 106.048192) (width 0.25) (layer B.Cu) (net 21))
 (segment (start 166.93 106.048192) (end 167.42 106.538192) (width 0.25) (layer B.Cu) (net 21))
 (segment (start 167.42 106.538192) (end 168.67 106.538192) (width 0.25) (layer B.Cu) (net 21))
 (segment (start 156.17 72.788192) (end 156.17 70.288192) (width 0.25) (layer B.Cu) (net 21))
 (segment (start 168.67 106.538192) (end 169.92 105.288192) (width 0.25) (layer B.Cu) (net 21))
 (segment (start 169.92 105.288192) (end 169.92 86.538192) (width 0.25) (layer B.Cu) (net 21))
 (segment (start 169.92 86.538192) (end 156.17 72.788192) (width 0.25) (layer B.Cu) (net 21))
 (segment (start 164.39 104.278192) (end 164.39 106.008192) (width 0.25) (layer B.Cu) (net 22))
 (segment (start 164.39 106.008192) (end 166.17 107.788192) (width 0.25) (layer B.Cu) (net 22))
 (segment (start 171.17 86.538192) (end 157.42 72.788192) (width 0.25) (layer B.Cu) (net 22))
 (segment (start 166.17 107.788192) (end 168.67 107.788192) (width 0.25) (layer B.Cu) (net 22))
 (segment (start 168.67 107.788192) (end 171.17 105.288192) (width 0.25) (layer B.Cu) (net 22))
 (segment (start 171.17 105.288192) (end 171.17 86.538192) (width 0.25) (layer B.Cu) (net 22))
 (segment (start 157.42 72.788192) (end 157.42 67.788192) (width 0.25) (layer B.Cu) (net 22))
 (segment (start 161.85 104.278192) (end 161.85 105.968192) (width 0.25) (layer B.Cu) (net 23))
 (segment (start 161.85 105.968192) (end 164.92 109.038192) (width 0.25) (layer B.Cu) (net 23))
 (segment (start 164.92 109.038192) (end 168.67 109.038192) (width 0.25) (layer B.Cu) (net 23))
 (segment (start 168.67 109.038192) (end 172.42 105.288192) (width 0.25) (layer B.Cu) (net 23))
 (segment (start 172.42 86.538192) (end 158.67 72.788192) (width 0.25) (layer B.Cu) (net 23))
 (segment (start 172.42 105.288192) (end 172.42 86.538192) (width 0.25) (layer B.Cu) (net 23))
 (segment (start 158.67 72.788192) (end 158.67 70.288192) (width 0.25) (layer B.Cu) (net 23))
 (segment (start 159.31 104.278192) (end 159.31 105.928192) (width 0.25) (layer B.Cu) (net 24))
 (segment (start 159.31 105.928192) (end 163.67 110.288192) (width 0.25) (layer B.Cu) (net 24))
 (segment (start 163.67 110.288192) (end 168.67 110.288192) (width 0.25) (layer B.Cu) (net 24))
 (segment (start 168.67 110.288192) (end 173.67 105.288192) (width 0.25) (layer B.Cu) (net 24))
 (segment (start 159.92 72.788192) (end 159.92 67.788192) (width 0.25) (layer B.Cu) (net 24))
 (segment (start 173.67 105.288192) (end 173.67 86.538192) (width 0.25) (layer B.Cu) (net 24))
 (segment (start 173.67 86.538192) (end 159.92 72.788192) (width 0.25) (layer B.Cu) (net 24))
 (segment (start 156.77 104.278192) (end 156.77 105.888192) (width 0.25) (layer B.Cu) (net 25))
 (segment (start 156.77 105.888192) (end 162.42 111.538192) (width 0.25) (layer B.Cu) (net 25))
 (segment (start 174.92 105.288192) (end 174.92 86.538192) (width 0.25) (layer B.Cu) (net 25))
 (segment (start 161.17 72.788192) (end 161.17 70.288192) (width 0.25) (layer B.Cu) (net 25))
 (segment (start 162.42 111.538192) (end 168.67 111.538192) (width 0.25) (layer B.Cu) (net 25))
 (segment (start 168.67 111.538192) (end 174.92 105.288192) (width 0.25) (layer B.Cu) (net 25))
 (segment (start 174.92 86.538192) (end 161.17 72.788192) (width 0.25) (layer B.Cu) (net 25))
 (segment (start 176.17 86.538192) (end 173.67 84.038192) (width 0.25) (layer B.Cu) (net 26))
 (segment (start 176.17 105.288192) (end 176.17 86.538192) (width 0.25) (layer B.Cu) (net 26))
 (segment (start 168.67 112.788192) (end 176.17 105.288192) (width 0.25) (layer B.Cu) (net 26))
 (segment (start 168.12712 112.788192) (end 168.67 112.788192) (width 0.25) (layer B.Cu) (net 26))
 (segment (start 161.17 112.788192) (end 168.12712 112.788192) (width 0.25) (layer B.Cu) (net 26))
 (segment (start 154.23 105.848192) (end 161.17 112.788192) (width 0.25) (layer B.Cu) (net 26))
 (segment (start 154.23 104.278192) (end 154.23 105.848192) (width 0.25) (layer B.Cu) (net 26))
 (segment (start 162.42 72.788192) (end 173.67 84.038192) (width 0.25) (layer B.Cu) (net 26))
 (segment (start 162.42 67.788192) (end 162.42 72.788192) (width 0.25) (layer B.Cu) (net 26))
 (segment (start 177.42 86.538192) (end 174.92 84.038192) (width 0.25) (layer B.Cu) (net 27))
 (segment (start 177.42 105.288192) (end 177.42 86.538192) (width 0.25) (layer B.Cu) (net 27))
 (segment (start 168.67 114.038192) (end 177.42 105.288192) (width 0.25) (layer B.Cu) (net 27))
 (segment (start 159.92 114.038192) (end 168.67 114.038192) (width 0.25) (layer B.Cu) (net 27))
 (segment (start 151.69 105.808192) (end 159.92 114.038192) (width 0.25) (layer B.Cu) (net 27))
 (segment (start 151.69 104.278192) (end 151.69 105.808192) (width 0.25) (layer B.Cu) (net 27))
 (segment (start 163.67 72.788192) (end 174.92 84.038192) (width 0.25) (layer B.Cu) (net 27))
 (segment (start 163.67 70.288192) (end 163.67 72.788192) (width 0.25) (layer B.Cu) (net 27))
 (segment (start 149.15 104.278192) (end 149.15 105.768192) (width 0.25) (layer B.Cu) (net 28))
 (segment (start 149.15 105.768192) (end 158.67 115.288192) (width 0.25) (layer B.Cu) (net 28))
 (segment (start 164.92 72.788192) (end 164.92 67.788192) (width 0.25) (layer B.Cu) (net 28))
 (segment (start 158.67 115.288192) (end 168.67 115.288192) (width 0.25) (layer B.Cu) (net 28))
 (segment (start 168.67 115.288192) (end 178.67 105.288192) (width 0.25) (layer B.Cu) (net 28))
 (segment (start 178.67 105.288192) (end 178.67 86.538192) (width 0.25) (layer B.Cu) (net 28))
 (segment (start 178.67 86.538192) (end 164.92 72.788192) (width 0.25) (layer B.Cu) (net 28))
 (segment (start 146.61 104.278192) (end 146.61 105.728192) (width 0.25) (layer B.Cu) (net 29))
 (segment (start 166.17 72.788192) (end 166.17 70.288192) (width 0.25) (layer B.Cu) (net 29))
 (segment (start 146.61 105.728192) (end 157.42 116.538192) (width 0.25) (layer B.Cu) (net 29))
 (segment (start 157.42 116.538192) (end 168.67 116.538192) (width 0.25) (layer B.Cu) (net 29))
 (segment (start 179.92 86.538192) (end 166.17 72.788192) (width 0.25) (layer B.Cu) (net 29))
 (segment (start 168.67 116.538192) (end 179.92 105.288192) (width 0.25) (layer B.Cu) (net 29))
 (segment (start 179.92 105.288192) (end 179.92 86.538192) (width 0.25) (layer B.Cu) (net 29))
 (segment (start 144.07 104.278192) (end 144.07 105.688192) (width 0.25) (layer B.Cu) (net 30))
 (segment (start 156.17 117.788192) (end 168.67 117.788192) (width 0.25) (layer B.Cu) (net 30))
 (segment (start 144.07 105.688192) (end 156.17 117.788192) (width 0.25) (layer B.Cu) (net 30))
 (segment (start 168.67 117.788192) (end 181.17 105.288192) (width 0.25) (layer B.Cu) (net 30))
 (segment (start 181.17 105.288192) (end 181.17 86.538192) (width 0.25) (layer B.Cu) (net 30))
 (segment (start 181.17 86.538192) (end 167.42 72.788192) (width 0.25) (layer B.Cu) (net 30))
 (segment (start 167.42 72.788192) (end 167.42 70.288192) (width 0.25) (layer B.Cu) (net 30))
 (segment (start 167.42 70.288192) (end 167.42 67.788192) (width 0.25) (layer B.Cu) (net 30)))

